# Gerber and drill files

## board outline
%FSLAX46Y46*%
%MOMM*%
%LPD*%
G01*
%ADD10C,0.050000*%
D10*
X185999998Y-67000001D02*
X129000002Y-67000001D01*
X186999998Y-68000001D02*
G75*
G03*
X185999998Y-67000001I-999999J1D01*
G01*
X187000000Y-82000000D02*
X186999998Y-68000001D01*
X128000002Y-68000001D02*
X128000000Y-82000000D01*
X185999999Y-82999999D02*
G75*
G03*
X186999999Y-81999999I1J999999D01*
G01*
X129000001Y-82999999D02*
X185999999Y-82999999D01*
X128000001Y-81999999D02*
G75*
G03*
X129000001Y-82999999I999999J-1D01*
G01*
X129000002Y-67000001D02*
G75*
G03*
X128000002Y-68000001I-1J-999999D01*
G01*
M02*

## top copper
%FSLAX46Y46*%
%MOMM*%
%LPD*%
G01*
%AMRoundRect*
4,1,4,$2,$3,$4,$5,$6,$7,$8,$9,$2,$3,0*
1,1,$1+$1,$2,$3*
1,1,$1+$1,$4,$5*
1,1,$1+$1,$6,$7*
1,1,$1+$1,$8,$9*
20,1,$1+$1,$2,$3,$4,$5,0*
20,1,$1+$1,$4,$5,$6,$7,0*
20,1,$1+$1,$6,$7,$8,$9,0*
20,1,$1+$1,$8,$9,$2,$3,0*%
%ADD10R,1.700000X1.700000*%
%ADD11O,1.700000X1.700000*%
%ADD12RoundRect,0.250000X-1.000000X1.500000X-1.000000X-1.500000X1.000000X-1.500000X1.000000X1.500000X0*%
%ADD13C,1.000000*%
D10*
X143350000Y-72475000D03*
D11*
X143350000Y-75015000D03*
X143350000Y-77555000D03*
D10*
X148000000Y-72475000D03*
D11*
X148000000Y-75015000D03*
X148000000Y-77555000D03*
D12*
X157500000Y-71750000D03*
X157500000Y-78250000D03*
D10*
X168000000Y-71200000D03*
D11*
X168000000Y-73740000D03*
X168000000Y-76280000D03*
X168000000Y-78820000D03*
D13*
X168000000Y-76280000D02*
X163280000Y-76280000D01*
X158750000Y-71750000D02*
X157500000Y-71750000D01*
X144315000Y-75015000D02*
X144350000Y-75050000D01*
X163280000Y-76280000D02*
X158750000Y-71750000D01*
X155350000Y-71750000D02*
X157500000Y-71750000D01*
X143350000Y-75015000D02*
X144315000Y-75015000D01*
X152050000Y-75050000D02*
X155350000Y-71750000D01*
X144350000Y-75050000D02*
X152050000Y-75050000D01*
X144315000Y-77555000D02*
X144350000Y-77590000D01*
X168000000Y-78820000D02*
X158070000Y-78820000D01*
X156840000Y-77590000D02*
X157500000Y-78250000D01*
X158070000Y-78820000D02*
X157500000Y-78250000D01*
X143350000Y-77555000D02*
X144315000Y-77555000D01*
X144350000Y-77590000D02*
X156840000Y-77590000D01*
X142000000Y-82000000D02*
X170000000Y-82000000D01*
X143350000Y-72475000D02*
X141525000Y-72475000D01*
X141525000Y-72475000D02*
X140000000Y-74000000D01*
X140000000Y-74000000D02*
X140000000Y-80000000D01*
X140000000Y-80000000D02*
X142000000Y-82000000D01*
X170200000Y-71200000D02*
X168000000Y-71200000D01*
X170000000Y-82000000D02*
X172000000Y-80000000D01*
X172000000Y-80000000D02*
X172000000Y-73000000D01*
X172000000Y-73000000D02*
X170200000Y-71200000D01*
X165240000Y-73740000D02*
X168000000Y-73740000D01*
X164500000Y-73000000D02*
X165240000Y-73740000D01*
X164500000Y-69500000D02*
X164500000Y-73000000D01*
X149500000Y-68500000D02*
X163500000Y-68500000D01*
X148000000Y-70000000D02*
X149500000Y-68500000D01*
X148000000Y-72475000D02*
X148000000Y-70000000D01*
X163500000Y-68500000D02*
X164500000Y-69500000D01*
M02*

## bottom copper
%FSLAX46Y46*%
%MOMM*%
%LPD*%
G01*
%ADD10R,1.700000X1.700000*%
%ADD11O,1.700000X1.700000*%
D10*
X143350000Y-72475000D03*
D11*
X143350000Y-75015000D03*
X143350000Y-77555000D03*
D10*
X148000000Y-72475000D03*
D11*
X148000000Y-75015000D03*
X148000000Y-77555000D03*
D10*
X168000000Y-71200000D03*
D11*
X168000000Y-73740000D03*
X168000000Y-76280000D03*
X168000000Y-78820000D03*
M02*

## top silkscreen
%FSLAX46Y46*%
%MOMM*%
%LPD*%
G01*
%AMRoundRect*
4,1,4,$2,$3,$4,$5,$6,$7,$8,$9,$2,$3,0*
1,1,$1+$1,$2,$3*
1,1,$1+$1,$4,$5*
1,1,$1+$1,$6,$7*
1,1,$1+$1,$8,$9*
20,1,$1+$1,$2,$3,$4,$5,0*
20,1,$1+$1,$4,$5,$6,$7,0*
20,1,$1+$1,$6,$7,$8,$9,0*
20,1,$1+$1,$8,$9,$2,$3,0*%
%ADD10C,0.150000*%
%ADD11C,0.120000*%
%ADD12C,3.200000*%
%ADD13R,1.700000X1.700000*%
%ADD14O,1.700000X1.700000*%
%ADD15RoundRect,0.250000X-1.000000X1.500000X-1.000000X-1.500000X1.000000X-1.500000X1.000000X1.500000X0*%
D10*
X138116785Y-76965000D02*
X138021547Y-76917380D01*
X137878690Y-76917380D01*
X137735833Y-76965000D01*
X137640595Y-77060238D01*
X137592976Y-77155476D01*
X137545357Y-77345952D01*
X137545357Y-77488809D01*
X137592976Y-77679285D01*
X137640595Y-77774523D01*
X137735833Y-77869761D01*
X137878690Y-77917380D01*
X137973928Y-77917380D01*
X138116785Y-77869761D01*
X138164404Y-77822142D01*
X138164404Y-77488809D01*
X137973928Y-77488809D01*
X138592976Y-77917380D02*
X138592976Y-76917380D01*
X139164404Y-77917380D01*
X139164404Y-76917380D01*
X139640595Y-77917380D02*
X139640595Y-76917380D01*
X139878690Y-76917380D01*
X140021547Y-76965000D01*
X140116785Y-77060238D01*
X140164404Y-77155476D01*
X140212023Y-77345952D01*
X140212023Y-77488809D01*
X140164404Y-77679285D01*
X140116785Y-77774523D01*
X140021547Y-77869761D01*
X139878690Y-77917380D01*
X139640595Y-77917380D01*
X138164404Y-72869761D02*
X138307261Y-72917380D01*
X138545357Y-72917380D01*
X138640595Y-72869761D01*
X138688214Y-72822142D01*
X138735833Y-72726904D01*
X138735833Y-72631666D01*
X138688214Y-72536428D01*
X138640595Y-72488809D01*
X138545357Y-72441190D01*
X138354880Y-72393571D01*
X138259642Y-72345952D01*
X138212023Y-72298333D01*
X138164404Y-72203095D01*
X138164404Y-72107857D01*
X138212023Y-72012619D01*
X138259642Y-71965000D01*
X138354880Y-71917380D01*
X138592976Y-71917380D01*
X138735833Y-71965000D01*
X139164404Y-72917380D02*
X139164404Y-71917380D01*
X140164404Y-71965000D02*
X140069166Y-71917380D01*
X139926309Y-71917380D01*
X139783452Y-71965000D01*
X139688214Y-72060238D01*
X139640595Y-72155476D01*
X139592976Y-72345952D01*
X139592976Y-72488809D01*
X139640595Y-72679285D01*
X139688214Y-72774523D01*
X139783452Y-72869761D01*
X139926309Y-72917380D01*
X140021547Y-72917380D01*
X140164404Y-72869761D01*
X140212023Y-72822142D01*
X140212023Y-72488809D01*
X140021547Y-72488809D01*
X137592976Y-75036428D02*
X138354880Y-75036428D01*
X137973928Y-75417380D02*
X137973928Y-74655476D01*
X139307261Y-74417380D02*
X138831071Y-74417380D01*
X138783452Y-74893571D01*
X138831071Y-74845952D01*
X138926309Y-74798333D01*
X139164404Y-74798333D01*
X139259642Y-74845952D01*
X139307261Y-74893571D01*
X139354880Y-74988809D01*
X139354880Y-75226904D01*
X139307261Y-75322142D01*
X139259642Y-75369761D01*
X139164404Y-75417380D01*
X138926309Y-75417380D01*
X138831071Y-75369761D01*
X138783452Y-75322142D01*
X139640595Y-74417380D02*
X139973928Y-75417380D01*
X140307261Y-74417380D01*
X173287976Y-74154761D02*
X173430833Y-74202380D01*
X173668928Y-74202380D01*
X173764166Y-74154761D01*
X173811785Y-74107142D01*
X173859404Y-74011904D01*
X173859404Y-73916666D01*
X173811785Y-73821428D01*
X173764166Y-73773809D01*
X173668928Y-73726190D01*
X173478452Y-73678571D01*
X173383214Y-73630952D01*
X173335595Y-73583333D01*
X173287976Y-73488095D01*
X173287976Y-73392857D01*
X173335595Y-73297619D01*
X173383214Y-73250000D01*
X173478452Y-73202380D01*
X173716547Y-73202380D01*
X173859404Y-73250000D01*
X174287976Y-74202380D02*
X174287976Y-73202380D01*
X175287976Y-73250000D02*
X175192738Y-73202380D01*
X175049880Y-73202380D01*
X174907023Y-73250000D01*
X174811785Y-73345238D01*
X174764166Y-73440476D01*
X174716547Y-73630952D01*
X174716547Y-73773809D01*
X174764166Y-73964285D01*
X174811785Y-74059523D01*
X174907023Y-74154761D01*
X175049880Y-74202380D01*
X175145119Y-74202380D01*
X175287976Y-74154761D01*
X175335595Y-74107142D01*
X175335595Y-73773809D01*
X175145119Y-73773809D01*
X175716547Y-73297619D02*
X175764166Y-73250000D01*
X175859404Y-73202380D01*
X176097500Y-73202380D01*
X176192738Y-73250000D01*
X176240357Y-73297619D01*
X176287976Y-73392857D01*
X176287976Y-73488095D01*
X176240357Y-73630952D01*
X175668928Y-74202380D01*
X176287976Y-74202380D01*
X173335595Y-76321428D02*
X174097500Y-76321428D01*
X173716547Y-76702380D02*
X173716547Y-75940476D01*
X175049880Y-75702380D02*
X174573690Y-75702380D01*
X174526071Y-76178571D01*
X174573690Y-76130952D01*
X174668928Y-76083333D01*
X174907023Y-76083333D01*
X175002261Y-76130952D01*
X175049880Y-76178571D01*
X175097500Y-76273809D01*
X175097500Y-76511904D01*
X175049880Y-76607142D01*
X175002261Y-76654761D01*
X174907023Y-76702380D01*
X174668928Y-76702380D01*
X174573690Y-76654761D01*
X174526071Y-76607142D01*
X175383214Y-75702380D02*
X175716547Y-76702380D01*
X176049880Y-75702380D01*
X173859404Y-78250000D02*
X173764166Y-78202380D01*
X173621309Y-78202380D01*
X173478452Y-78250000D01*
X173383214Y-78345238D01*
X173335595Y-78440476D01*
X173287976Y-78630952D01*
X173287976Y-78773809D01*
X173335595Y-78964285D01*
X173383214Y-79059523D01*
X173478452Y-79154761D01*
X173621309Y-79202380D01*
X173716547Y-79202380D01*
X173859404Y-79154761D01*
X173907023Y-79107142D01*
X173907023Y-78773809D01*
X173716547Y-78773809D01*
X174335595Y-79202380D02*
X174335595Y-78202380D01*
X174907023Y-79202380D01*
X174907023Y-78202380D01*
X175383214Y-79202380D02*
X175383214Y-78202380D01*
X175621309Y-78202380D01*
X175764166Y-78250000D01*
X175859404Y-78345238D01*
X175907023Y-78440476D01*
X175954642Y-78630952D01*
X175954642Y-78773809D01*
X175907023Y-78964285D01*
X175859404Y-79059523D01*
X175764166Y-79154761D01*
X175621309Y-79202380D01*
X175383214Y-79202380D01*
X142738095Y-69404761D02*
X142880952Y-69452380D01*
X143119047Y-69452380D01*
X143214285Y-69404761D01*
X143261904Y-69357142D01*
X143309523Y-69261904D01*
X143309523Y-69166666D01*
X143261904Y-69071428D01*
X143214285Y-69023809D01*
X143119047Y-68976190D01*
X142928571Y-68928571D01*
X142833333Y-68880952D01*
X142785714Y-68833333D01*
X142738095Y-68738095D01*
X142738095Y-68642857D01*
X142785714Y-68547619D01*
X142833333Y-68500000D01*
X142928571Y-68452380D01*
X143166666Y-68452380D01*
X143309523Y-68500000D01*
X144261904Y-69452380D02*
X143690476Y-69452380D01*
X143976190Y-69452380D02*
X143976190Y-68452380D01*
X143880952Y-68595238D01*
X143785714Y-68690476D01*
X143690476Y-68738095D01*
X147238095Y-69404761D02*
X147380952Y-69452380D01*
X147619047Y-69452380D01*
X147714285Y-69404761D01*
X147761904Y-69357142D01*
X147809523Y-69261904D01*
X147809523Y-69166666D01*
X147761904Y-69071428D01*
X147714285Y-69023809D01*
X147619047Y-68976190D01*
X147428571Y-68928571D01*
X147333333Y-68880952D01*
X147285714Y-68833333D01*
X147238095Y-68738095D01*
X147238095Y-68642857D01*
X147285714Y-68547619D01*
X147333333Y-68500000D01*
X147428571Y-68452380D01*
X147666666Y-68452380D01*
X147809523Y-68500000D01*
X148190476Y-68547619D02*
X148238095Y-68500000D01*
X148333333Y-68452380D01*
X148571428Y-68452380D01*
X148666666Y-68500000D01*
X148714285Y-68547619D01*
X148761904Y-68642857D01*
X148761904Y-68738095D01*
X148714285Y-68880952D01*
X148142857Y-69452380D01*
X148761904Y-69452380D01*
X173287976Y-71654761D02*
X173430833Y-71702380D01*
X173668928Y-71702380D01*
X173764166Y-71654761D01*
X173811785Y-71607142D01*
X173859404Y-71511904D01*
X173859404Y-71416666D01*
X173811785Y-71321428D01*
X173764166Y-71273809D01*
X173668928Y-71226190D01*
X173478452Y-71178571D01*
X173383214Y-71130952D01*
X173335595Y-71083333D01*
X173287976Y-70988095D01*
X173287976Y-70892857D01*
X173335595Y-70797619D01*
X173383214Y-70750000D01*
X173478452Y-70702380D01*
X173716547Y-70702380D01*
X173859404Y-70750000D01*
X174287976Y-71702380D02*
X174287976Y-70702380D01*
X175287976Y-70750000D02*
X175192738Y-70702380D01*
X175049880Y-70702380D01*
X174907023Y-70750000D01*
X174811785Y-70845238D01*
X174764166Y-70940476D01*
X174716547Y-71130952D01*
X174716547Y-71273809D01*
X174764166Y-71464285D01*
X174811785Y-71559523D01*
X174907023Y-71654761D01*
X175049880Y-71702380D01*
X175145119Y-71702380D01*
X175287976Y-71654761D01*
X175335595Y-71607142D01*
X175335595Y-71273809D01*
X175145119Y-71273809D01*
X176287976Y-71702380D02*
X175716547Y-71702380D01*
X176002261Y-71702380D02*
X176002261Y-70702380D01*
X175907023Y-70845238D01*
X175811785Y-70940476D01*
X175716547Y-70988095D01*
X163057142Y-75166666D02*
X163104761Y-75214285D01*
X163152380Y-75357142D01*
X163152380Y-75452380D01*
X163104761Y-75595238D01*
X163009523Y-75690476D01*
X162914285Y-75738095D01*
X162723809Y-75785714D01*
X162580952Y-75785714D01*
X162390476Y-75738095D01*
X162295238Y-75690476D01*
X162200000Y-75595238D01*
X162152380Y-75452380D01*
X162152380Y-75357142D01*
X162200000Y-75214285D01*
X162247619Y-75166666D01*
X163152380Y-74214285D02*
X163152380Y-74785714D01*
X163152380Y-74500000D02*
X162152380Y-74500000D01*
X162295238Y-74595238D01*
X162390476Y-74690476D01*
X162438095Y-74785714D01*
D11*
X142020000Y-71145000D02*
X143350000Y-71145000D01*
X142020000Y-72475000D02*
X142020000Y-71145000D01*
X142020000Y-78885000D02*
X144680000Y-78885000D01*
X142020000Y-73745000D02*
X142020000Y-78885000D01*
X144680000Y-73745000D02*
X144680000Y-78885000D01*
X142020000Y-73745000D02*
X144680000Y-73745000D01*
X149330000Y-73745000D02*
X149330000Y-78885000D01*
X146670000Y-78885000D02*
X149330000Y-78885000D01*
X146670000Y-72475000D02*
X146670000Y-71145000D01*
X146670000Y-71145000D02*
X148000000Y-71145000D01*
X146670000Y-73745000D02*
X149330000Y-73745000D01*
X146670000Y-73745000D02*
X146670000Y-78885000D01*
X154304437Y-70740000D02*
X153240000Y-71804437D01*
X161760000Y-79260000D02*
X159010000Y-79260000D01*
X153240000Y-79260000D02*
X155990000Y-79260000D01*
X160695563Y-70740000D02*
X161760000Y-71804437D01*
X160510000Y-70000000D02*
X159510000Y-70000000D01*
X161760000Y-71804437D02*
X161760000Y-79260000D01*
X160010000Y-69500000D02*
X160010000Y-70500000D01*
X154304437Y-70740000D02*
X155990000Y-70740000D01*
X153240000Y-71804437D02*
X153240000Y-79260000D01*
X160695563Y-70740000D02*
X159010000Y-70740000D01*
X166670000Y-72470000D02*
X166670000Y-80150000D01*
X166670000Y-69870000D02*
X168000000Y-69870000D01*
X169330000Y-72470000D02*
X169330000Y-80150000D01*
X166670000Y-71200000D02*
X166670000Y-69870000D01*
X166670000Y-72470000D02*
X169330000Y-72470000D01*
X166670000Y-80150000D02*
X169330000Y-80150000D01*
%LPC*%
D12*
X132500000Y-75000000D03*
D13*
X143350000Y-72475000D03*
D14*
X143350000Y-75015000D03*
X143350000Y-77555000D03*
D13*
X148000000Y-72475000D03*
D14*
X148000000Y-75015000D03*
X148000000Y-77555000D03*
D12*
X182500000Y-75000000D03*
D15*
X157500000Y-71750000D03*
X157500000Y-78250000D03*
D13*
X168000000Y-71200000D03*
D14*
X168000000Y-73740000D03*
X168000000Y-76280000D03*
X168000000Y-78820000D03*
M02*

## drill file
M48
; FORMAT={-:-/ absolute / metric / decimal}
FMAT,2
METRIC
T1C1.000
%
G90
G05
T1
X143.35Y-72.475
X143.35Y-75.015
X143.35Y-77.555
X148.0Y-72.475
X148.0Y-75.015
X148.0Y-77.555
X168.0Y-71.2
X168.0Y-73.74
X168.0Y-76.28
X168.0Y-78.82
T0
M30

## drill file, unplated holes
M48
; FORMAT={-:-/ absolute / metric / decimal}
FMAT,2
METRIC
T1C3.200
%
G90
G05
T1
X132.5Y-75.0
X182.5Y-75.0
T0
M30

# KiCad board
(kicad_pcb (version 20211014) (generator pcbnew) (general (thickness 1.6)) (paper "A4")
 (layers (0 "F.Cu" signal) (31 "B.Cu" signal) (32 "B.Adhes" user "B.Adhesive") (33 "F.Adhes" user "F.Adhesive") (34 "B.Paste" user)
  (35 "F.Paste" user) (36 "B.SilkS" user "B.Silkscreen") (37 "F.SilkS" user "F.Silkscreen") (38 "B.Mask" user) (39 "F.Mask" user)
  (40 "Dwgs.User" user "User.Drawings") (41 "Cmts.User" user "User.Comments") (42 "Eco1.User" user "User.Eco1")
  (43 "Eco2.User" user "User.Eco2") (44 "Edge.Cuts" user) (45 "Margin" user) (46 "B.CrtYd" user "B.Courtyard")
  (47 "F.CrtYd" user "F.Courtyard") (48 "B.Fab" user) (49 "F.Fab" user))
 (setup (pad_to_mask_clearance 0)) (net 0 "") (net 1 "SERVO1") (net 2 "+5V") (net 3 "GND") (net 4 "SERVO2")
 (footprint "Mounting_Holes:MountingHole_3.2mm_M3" (layer "F.Cu") (at 132.5 75)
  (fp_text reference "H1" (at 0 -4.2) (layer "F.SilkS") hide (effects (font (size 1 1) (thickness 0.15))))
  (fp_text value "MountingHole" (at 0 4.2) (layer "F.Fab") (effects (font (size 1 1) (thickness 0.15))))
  (pad "" np_thru_hole circle locked (at 0 0) (size 3.2 3.2) (drill 3.2) (layers *.Cu *.Mask)))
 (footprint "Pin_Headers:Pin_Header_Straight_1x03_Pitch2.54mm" (layer "F.Cu") (at 143.35 72.475)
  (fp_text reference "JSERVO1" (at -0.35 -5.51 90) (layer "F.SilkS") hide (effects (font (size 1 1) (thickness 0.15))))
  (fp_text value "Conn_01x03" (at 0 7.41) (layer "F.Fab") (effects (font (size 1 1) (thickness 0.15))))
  (fp_line (start -1.33 -1.33) (end 0 -1.33) (layer "F.SilkS") (width 0.12))
  (fp_line (start -1.33 0) (end -1.33 -1.33) (layer "F.SilkS") (width 0.12))
  (fp_line (start -1.33 6.41) (end 1.33 6.41) (layer "F.SilkS") (width 0.12))
  (fp_line (start -1.33 1.27) (end -1.33 6.41) (layer "F.SilkS") (width 0.12))
  (fp_line (start 1.33 1.27) (end 1.33 6.41) (layer "F.SilkS") (width 0.12))
  (fp_line (start -1.33 1.27) (end 1.33 1.27) (layer "F.SilkS") (width 0.12))
  (pad "1" thru_hole rect locked (at 0 0) (size 1.7 1.7) (drill 1) (layers *.Cu *.Mask) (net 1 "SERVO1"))
  (pad "2" thru_hole oval locked (at 0 2.54) (size 1.7 1.7) (drill 1) (layers *.Cu *.Mask) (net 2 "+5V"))
  (pad "3" thru_hole oval locked (at 0 5.08) (size 1.7 1.7) (drill 1) (layers *.Cu *.Mask) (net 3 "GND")))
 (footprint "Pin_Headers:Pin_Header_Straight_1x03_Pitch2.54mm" (layer "F.Cu") (at 148 72.475)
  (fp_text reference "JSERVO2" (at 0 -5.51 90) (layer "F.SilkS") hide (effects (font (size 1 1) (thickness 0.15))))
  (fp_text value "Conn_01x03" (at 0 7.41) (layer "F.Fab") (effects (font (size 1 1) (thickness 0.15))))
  (fp_line (start 1.33 1.27) (end 1.33 6.41) (layer "F.SilkS") (width 0.12))
  (fp_line (start -1.33 6.41) (end 1.33 6.41) (layer "F.SilkS") (width 0.12))
  (fp_line (start -1.33 0) (end -1.33 -1.33) (layer "F.SilkS") (width 0.12))
  (fp_line (start -1.33 -1.33) (end 0 -1.33) (layer "F.SilkS") (width 0.12))
  (fp_line (start -1.33 1.27) (end 1.33 1.27) (layer "F.SilkS") (width 0.12))
  (fp_line (start -1.33 1.27) (end -1.33 6.41) (layer "F.SilkS") (width 0.12))
  (pad "1" thru_hole rect locked (at 0 0) (size 1.7 1.7) (drill 1) (layers *.Cu *.Mask) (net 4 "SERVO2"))
  (pad "2" thru_hole oval locked (at 0 2.54) (size 1.7 1.7) (drill 1) (layers *.Cu *.Mask) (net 2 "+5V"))
  (pad "3" thru_hole oval locked (at 0 5.08) (size 1.7 1.7) (drill 1) (layers *.Cu *.Mask) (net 3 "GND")))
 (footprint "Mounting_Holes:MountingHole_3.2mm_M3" (layer "F.Cu") (at 182.5 75)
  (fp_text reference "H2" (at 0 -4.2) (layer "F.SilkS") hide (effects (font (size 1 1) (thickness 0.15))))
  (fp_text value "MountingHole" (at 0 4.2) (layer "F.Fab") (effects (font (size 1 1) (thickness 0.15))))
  (pad "" np_thru_hole circle locked (at 0 0) (size 3.2 3.2) (drill 3.2) (layers *.Cu *.Mask)))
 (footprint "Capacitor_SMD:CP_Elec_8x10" (layer "F.Cu") (at 157.5 75 -90)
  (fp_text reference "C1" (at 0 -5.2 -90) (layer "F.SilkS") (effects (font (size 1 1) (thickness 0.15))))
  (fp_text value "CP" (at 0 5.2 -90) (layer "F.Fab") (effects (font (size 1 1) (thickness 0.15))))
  (fp_line (start -4.26 3.195563) (end -3.195563 4.26) (layer "F.SilkS") (width 0.12))
  (fp_line (start 4.26 -4.26) (end 4.26 -1.51) (layer "F.SilkS") (width 0.12))
  (fp_line (start 4.26 4.26) (end 4.26 1.51) (layer "F.SilkS") (width 0.12))
  (fp_line (start -4.26 -3.195563) (end -3.195563 -4.26) (layer "F.SilkS") (width 0.12))
  (fp_line (start -5 -3.01) (end -5 -2.01) (layer "F.SilkS") (width 0.12))
  (fp_line (start -3.195563 -4.26) (end 4.26 -4.26) (layer "F.SilkS") (width 0.12))
  (fp_line (start -5.5 -2.51) (end -4.5 -2.51) (layer "F.SilkS") (width 0.12))
  (fp_line (start -4.26 3.195563) (end -4.26 1.51) (layer "F.SilkS") (width 0.12))
  (fp_line (start -3.195563 4.26) (end 4.26 4.26) (layer "F.SilkS") (width 0.12))
  (fp_line (start -4.26 -3.195563) (end -4.26 -1.51) (layer "F.SilkS") (width 0.12))
  (pad "1" smd roundrect locked (at -3.25 0 270) (size 3.5 2.5) (layers "F.Cu" "F.Paste" "F.Mask") (roundrect_rratio 0.1) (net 2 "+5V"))
  (pad "2" smd roundrect locked (at 3.25 0 270) (size 3.5 2.5) (layers "F.Cu" "F.Paste" "F.Mask") (roundrect_rratio 0.1) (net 3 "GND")))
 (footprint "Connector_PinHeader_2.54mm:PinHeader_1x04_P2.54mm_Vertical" (layer "F.Cu") (at 168 71.2)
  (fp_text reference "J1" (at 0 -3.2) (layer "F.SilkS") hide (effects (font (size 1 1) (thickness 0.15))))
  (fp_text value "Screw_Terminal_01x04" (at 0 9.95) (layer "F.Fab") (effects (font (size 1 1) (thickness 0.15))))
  (fp_line (start -1.33 1.27) (end -1.33 8.95) (layer "F.SilkS") (width 0.12))
  (fp_line (start -1.33 -1.33) (end 0 -1.33) (layer "F.SilkS") (width 0.12))
  (fp_line (start 1.33 1.27) (end 1.33 8.95) (layer "F.SilkS") (width 0.12))
  (fp_line (start -1.33 0) (end -1.33 -1.33) (layer "F.SilkS") (width 0.12))
  (fp_line (start -1.33 1.27) (end 1.33 1.27) (layer "F.SilkS") (width 0.12))
  (fp_line (start -1.33 8.95) (end 1.33 8.95) (layer "F.SilkS") (width 0.12))
  (pad "1" thru_hole rect locked (at 0 0) (size 1.7 1.7) (drill 1) (layers *.Cu *.Mask) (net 1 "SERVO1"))
  (pad "2" thru_hole oval locked (at 0 2.54) (size 1.7 1.7) (drill 1) (layers *.Cu *.Mask) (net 4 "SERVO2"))
  (pad "3" thru_hole oval locked (at 0 5.08) (size 1.7 1.7) (drill 1) (layers *.Cu *.Mask) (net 2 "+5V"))
  (pad "4" thru_hole oval locked (at 0 7.62) (size 1.7 1.7) (drill 1) (layers *.Cu *.Mask) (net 3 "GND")))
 (gr_line (start 185.999998 67.000001) (end 129.000002 67.000001) (layer "Edge.Cuts") (width 0.05))
 (gr_arc (start 185.999998 67.000001) (mid 186.707105 67.292894) (end 186.999998 68.000001) (layer "Edge.Cuts") (width 0.05))
 (gr_line (start 187 82) (end 186.999998 68.000001) (layer "Edge.Cuts") (width 0.05))
 (gr_line (start 128.000002 68.000001) (end 128 82) (layer "Edge.Cuts") (width 0.05))
 (gr_arc (start 186.999999 81.999999) (mid 186.707106 82.707106) (end 185.999999 82.999999) (layer "Edge.Cuts") (width 0.05))
 (gr_line (start 129.000001 82.999999) (end 185.999999 82.999999) (layer "Edge.Cuts") (width 0.05))
 (gr_arc (start 129.000001 82.999999) (mid 128.292894 82.707106) (end 128.000001 81.999999) (layer "Edge.Cuts") (width 0.05))
 (gr_arc (start 128.000002 68.000001) (mid 128.292895 67.292894) (end 129.000002 67.000001) (layer "Edge.Cuts") (width 0.05))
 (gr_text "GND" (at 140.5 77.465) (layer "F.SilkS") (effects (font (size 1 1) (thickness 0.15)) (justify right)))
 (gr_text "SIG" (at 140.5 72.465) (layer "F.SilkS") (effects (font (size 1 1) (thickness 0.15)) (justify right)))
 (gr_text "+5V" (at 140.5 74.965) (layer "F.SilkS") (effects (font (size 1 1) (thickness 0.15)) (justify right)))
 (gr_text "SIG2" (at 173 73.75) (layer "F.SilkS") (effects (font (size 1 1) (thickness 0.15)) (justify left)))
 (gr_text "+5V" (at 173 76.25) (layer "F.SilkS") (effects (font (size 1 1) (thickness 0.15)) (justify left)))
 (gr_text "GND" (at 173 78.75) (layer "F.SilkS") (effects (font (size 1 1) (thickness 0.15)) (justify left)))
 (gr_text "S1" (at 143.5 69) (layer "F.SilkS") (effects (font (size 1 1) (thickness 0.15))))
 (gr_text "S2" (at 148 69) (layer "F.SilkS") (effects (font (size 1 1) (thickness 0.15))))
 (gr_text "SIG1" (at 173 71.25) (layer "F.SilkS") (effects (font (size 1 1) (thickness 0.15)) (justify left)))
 (segment (start 168 76.28) (end 163.28 76.28) (width 1) (layer "F.Cu") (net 2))
 (segment (start 158.75 71.75) (end 157.5 71.75) (width 1) (layer "F.Cu") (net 2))
 (segment (start 144.315 75.015) (end 144.35 75.05) (width 1) (layer "F.Cu") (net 2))
 (segment (start 163.28 76.28) (end 158.75 71.75) (width 1) (layer "F.Cu") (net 2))
 (segment (start 155.35 71.75) (end 157.5 71.75) (width 1) (layer "F.Cu") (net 2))
 (segment (start 143.35 75.015) (end 144.315 75.015) (width 1) (layer "F.Cu") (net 2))
 (segment (start 152.05 75.05) (end 155.35 71.75) (width 1) (layer "F.Cu") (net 2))
 (segment (start 144.35 75.05) (end 152.05 75.05) (width 1) (layer "F.Cu") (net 2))
 (segment (start 144.315 77.555) (end 144.35 77.59) (width 1) (layer "F.Cu") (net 3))
 (segment (start 168 78.82) (end 158.07 78.82) (width 1) (layer "F.Cu") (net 3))
 (segment (start 156.84 77.59) (end 157.5 78.25) (width 1) (layer "F.Cu") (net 3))
 (segment (start 158.07 78.82) (end 157.5 78.25) (width 1) (layer "F.Cu") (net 3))
 (segment (start 143.35 77.555) (end 144.315 77.555) (width 1) (layer "F.Cu") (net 3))
 (segment (start 144.35 77.59) (end 156.84 77.59) (width 1) (layer "F.Cu") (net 3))
 (segment (start 142 82) (end 170 82) (width 1) (layer "F.Cu") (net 1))
 (segment (start 143.35 72.475) (end 141.525 72.475) (width 1) (layer "F.Cu") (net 1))
 (segment (start 141.525 72.475) (end 140 74) (width 1) (layer "F.Cu") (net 1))
 (segment (start 140 74) (end 140 80) (width 1) (layer "F.Cu") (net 1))
 (segment (start 140 80) (end 142 82) (width 1) (layer "F.Cu") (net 1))
 (segment (start 170.2 71.2) (end 168 71.2) (width 1) (layer "F.Cu") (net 1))
 (segment (start 170 82) (end 172 80) (width 1) (layer "F.Cu") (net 1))
 (segment (start 172 80) (end 172 73) (width 1) (layer "F.Cu") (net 1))
 (segment (start 172 73) (end 170.2 71.2) (width 1) (layer "F.Cu") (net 1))
 (segment (start 165.24 73.74) (end 168 73.74) (width 1) (layer "F.Cu") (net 4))
 (segment (start 164.5 73) (end 165.24 73.74) (width 1) (layer "F.Cu") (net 4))
 (segment (start 164.5 69.5) (end 164.5 73) (width 1) (layer "F.Cu") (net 4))
 (segment (start 149.5 68.5) (end 163.5 68.5) (width 1) (layer "F.Cu") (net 4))
 (segment (start 148 70) (end 149.5 68.5) (width 1) (layer "F.Cu") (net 4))
 (segment (start 148 72.475) (end 148 70) (width 1) (layer "F.Cu") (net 4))
 (segment (start 163.5 68.5) (end 164.5 69.5) (width 1) (layer "F.Cu") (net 4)))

